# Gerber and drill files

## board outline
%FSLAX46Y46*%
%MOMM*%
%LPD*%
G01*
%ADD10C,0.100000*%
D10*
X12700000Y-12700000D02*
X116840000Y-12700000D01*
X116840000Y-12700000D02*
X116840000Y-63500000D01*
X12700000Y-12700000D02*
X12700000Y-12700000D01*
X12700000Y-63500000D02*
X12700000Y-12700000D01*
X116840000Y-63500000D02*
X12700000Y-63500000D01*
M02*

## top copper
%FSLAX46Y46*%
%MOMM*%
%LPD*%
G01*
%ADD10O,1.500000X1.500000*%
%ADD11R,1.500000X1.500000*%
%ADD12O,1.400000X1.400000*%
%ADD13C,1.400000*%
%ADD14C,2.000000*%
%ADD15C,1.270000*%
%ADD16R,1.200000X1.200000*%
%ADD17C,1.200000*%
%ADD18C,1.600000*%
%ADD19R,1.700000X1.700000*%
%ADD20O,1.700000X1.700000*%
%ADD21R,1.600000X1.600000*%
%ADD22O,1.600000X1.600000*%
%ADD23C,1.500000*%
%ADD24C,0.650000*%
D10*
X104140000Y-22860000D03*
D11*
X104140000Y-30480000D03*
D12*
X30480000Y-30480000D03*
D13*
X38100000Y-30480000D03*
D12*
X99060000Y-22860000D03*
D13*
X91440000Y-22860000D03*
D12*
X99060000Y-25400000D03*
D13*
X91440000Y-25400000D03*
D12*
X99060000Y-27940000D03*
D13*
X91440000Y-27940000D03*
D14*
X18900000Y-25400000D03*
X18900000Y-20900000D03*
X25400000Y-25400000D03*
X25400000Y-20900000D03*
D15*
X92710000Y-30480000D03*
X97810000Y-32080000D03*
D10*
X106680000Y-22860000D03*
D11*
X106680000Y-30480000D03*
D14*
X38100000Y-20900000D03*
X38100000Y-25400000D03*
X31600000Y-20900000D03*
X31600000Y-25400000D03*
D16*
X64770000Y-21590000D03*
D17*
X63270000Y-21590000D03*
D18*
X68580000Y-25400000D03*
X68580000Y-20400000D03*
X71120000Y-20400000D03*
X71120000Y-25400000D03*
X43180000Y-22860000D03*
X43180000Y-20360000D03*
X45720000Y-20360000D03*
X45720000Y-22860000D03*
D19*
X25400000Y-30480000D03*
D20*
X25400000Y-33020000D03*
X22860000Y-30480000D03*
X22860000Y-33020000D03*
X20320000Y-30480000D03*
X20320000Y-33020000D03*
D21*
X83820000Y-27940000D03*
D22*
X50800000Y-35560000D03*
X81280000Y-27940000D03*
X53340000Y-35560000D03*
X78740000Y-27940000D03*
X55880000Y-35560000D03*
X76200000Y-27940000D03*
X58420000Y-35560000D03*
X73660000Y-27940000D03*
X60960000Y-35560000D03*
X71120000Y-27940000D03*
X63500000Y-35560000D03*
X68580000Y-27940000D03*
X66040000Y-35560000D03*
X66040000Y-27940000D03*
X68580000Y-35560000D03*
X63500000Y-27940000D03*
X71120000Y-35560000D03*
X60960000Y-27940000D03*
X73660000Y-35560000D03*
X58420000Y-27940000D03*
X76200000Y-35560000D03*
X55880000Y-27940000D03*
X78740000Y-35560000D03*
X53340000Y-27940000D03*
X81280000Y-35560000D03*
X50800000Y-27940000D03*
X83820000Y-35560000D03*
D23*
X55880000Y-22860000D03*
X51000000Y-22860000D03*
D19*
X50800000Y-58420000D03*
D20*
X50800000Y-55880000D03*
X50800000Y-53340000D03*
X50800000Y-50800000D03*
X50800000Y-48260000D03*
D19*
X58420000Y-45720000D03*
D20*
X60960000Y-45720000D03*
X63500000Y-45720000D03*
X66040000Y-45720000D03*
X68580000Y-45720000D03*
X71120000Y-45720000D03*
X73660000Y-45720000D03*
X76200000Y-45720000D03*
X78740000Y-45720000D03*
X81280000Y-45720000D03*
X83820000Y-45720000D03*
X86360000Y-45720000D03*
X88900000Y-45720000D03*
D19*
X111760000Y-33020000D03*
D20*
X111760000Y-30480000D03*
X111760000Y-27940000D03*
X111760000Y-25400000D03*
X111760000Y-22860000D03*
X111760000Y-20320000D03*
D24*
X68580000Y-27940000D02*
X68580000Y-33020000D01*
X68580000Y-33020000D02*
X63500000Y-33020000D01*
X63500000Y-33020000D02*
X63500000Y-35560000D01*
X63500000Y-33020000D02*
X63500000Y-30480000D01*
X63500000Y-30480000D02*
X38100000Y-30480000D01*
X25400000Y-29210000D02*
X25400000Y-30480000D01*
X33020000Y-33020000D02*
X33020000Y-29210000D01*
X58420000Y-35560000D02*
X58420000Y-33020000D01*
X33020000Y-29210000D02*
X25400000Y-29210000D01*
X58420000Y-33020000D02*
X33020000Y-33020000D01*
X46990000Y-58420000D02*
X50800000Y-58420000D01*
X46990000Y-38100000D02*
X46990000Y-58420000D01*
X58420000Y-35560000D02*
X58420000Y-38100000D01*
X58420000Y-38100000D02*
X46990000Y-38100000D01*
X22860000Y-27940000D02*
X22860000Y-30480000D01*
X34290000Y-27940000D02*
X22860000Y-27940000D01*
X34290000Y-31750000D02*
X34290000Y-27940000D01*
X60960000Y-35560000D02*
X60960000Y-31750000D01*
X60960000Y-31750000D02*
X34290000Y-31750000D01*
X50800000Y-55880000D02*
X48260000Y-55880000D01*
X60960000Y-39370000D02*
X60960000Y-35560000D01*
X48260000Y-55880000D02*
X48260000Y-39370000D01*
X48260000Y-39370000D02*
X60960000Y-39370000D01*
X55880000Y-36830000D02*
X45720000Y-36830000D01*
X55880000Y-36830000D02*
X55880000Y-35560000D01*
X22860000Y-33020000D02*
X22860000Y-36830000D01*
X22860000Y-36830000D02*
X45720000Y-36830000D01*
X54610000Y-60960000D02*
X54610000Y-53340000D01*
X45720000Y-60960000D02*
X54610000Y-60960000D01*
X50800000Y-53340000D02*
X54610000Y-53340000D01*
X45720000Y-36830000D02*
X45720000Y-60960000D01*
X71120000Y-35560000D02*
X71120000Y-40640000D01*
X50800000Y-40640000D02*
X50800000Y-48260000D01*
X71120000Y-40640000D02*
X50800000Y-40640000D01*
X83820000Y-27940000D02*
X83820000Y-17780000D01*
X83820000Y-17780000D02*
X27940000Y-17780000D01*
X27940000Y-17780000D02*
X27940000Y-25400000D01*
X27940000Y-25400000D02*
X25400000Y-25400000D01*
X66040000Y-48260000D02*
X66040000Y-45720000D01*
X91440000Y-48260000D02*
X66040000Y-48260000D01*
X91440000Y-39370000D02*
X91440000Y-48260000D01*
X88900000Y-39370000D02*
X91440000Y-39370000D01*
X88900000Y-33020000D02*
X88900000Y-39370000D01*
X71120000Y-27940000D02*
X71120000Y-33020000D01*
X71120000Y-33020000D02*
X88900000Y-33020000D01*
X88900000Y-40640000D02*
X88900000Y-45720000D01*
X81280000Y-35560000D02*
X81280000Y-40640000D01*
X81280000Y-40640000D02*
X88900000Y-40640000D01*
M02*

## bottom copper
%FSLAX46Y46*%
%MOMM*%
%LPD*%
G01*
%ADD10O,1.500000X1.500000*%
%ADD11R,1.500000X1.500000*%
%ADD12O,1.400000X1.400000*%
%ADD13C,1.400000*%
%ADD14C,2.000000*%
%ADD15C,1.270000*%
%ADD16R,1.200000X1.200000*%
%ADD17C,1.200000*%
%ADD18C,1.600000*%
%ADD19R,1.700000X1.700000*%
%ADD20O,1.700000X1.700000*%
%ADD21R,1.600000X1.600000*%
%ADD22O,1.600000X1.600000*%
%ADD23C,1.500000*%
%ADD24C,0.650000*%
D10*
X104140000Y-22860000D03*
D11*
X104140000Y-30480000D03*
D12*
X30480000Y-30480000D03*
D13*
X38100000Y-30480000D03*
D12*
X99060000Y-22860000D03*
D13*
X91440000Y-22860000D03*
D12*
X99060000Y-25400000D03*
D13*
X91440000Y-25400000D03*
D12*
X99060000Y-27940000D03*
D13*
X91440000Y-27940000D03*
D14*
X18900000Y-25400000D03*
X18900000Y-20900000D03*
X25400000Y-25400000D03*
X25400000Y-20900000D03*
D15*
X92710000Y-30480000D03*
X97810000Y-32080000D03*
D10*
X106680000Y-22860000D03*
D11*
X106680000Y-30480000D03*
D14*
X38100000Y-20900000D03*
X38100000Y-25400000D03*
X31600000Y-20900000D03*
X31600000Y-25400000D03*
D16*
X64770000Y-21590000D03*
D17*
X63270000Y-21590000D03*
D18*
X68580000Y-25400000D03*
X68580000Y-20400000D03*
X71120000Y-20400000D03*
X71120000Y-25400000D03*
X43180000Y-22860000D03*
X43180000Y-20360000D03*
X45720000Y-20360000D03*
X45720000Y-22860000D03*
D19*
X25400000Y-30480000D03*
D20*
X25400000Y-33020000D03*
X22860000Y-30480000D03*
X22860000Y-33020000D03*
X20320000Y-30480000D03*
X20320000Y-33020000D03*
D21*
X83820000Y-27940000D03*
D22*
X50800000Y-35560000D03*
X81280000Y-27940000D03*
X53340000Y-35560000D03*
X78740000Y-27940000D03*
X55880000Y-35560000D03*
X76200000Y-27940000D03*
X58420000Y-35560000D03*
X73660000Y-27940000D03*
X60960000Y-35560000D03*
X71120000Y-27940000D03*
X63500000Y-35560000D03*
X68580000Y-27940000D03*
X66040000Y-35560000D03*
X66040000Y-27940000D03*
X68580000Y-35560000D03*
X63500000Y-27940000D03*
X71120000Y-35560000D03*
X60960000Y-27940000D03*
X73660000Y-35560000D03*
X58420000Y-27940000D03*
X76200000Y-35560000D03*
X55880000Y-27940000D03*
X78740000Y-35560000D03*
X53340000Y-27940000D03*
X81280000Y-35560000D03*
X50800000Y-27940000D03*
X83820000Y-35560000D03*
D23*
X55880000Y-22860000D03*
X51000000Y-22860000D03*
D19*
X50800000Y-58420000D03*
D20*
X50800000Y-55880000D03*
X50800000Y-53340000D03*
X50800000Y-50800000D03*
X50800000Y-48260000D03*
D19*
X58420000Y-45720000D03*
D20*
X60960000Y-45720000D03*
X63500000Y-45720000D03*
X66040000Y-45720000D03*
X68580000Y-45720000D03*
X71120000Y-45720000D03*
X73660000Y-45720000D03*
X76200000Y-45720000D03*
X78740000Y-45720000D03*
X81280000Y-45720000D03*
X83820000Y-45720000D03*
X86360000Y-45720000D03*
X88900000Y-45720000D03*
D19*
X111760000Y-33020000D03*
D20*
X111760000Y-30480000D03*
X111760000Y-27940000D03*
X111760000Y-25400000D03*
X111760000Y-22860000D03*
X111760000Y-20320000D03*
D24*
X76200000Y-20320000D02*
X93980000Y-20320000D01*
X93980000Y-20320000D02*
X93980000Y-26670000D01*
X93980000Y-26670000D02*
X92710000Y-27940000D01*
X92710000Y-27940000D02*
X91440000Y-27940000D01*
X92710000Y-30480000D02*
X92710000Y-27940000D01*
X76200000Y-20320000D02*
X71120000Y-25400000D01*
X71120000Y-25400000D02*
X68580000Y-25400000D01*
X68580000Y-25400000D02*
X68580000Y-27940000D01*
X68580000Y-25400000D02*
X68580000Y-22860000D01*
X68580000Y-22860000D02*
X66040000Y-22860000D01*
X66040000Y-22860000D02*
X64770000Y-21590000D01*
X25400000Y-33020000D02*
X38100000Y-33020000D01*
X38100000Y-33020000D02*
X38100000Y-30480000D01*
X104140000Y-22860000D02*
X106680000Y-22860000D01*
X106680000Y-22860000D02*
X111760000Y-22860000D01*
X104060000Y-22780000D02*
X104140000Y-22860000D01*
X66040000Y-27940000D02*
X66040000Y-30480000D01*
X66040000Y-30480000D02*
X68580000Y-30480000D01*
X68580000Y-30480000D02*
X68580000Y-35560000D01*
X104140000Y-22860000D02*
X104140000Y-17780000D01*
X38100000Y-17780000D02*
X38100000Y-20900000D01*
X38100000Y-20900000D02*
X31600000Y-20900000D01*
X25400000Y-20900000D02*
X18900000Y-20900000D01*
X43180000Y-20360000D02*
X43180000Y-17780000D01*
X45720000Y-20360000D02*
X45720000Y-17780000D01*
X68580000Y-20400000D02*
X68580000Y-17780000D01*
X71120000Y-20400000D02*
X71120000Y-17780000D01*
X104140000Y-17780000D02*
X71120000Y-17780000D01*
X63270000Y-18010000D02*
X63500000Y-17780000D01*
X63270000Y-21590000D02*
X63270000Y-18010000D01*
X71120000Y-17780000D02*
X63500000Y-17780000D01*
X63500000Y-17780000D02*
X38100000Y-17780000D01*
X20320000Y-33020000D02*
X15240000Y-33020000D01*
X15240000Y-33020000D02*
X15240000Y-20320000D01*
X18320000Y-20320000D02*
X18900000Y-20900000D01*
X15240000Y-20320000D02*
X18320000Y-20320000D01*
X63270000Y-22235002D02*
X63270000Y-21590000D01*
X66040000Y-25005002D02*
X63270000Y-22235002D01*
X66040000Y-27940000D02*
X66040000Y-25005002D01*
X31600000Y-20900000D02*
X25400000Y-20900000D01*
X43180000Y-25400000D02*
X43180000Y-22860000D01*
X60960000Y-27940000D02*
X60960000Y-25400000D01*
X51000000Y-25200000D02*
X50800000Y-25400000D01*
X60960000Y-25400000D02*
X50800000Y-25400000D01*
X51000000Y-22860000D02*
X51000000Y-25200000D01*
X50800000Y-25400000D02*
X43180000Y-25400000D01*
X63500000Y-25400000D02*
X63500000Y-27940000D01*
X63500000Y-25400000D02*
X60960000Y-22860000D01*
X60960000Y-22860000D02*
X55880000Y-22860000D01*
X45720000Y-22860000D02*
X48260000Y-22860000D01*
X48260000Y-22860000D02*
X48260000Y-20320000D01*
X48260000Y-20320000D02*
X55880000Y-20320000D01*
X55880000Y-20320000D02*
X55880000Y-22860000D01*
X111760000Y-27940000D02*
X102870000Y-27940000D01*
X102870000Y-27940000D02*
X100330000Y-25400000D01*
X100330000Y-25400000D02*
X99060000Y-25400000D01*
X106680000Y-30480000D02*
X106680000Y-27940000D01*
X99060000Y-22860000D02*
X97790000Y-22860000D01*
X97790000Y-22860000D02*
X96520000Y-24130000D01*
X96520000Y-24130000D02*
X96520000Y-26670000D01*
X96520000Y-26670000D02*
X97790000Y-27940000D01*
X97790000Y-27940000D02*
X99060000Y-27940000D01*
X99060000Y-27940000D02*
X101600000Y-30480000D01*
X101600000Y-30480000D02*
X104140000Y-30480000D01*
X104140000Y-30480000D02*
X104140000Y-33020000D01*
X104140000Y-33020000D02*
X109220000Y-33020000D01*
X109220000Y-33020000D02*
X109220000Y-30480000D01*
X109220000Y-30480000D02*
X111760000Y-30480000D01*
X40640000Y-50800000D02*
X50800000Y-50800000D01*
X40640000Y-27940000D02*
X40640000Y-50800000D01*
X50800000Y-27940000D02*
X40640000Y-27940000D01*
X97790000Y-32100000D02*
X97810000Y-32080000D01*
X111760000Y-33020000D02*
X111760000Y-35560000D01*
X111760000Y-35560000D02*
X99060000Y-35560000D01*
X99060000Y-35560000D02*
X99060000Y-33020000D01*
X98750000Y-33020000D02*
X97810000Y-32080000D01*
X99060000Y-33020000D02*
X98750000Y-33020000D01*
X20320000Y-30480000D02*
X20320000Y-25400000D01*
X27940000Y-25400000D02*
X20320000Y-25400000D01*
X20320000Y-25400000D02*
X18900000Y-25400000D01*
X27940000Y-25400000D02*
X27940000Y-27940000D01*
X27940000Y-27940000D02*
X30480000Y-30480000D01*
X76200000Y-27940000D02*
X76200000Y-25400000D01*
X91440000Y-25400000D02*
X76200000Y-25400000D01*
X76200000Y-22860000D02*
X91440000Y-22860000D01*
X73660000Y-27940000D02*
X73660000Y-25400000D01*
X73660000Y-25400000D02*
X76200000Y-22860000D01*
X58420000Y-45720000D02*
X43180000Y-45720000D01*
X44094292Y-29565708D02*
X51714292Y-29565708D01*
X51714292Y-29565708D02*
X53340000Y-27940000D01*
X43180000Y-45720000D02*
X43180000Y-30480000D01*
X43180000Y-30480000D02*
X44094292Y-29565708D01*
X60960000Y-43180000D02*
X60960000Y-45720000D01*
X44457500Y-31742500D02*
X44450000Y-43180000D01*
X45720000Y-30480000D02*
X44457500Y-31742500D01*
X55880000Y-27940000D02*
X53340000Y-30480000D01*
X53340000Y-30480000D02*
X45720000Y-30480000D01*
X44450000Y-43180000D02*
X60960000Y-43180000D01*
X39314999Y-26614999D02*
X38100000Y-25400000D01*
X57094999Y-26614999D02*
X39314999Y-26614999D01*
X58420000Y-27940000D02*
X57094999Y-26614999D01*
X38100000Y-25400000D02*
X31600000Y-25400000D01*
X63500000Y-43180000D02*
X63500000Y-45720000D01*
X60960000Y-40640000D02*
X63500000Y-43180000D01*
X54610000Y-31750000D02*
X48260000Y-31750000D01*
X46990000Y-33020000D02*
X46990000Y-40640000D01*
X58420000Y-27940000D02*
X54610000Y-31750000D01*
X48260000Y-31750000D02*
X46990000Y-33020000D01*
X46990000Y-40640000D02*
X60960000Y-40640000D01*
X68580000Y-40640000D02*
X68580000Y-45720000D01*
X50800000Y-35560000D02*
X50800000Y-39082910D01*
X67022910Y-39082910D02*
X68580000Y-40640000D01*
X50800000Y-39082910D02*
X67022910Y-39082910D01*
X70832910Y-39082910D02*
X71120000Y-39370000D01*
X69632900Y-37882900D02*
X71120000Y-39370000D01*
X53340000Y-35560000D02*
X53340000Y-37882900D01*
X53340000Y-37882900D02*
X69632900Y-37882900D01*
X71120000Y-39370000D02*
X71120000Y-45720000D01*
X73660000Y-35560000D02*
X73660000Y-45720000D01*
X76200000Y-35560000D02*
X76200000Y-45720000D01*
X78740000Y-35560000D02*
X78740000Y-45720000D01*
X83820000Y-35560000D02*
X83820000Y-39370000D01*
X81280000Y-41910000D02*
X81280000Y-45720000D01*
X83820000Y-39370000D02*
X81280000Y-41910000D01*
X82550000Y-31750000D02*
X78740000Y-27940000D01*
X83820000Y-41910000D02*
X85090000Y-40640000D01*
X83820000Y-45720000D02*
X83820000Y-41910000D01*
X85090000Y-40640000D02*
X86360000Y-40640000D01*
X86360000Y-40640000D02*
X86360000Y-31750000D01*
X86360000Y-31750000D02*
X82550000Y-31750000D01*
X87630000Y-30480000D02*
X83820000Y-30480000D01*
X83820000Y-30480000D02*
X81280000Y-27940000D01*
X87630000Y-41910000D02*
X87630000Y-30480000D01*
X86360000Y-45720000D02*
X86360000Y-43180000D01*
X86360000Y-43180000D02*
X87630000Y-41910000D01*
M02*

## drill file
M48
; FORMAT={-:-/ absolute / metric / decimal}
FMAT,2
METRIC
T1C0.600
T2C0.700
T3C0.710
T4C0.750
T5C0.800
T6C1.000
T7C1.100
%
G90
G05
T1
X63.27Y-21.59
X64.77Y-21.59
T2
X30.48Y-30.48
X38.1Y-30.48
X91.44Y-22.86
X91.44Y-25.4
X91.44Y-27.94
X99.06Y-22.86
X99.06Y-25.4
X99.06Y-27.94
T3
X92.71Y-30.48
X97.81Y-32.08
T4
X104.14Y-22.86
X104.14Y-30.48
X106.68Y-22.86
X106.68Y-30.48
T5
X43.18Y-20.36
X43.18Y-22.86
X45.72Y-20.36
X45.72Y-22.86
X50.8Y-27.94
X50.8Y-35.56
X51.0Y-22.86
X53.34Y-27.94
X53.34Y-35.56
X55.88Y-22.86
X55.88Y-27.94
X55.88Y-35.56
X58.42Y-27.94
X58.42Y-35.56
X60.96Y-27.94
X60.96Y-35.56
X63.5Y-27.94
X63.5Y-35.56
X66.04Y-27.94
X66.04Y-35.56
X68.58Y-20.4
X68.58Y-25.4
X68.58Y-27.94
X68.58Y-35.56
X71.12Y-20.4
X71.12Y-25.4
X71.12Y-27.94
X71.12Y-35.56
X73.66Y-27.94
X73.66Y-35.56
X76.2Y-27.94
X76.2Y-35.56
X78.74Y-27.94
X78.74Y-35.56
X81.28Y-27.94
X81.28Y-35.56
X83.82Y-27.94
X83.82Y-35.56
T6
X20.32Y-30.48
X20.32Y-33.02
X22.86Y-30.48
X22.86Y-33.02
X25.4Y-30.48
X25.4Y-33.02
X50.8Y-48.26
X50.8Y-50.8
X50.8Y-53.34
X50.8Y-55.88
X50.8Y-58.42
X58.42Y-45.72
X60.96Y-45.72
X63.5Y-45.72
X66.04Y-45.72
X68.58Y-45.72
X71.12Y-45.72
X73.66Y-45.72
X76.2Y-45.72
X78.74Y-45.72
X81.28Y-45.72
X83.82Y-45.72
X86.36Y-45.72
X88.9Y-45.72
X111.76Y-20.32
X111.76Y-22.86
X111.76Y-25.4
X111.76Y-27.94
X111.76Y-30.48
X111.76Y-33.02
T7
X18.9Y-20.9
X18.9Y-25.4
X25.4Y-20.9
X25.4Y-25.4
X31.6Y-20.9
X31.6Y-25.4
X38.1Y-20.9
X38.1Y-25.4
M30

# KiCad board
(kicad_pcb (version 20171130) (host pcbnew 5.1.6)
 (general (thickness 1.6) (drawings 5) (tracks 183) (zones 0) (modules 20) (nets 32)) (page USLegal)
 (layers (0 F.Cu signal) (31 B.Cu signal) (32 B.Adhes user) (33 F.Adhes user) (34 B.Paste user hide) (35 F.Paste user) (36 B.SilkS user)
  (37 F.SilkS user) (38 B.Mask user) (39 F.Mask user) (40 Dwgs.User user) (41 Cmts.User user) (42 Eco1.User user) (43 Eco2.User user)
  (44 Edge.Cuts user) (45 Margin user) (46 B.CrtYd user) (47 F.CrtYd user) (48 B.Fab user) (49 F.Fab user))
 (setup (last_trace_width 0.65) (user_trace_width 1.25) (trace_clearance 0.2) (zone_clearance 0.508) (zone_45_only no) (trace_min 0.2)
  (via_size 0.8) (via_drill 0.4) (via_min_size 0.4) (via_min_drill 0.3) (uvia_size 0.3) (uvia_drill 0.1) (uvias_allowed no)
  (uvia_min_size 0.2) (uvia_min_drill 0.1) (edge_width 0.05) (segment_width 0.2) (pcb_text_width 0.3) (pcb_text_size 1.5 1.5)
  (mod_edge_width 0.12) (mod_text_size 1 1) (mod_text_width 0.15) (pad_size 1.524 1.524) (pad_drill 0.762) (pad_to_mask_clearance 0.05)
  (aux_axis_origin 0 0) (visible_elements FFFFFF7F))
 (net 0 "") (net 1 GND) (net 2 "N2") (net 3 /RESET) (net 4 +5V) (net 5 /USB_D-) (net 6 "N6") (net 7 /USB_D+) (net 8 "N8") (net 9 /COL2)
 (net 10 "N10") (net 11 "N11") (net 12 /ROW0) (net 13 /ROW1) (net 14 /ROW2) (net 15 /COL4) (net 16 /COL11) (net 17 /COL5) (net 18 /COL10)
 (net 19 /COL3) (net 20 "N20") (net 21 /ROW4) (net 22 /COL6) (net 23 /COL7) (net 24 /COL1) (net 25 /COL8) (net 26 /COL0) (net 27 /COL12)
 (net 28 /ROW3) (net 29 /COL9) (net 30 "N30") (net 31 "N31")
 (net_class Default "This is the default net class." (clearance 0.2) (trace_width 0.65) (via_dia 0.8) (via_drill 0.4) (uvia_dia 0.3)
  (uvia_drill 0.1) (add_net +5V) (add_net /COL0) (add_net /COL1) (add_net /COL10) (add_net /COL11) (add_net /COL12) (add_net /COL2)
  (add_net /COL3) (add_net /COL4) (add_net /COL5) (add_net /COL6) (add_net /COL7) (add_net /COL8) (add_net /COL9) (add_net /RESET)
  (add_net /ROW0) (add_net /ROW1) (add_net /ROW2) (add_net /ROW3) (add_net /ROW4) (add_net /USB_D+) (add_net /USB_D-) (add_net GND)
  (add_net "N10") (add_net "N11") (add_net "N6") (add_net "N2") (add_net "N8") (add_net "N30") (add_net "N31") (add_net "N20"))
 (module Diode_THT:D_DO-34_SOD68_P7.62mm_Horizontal (layer F.Cu) (at 104.14 30.48 90)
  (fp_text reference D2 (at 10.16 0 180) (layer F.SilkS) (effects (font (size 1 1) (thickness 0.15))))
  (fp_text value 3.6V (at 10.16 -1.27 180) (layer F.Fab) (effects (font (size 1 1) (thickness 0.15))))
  (pad 2 thru_hole oval (at 7.62 0 90) (size 1.5 1.5) (drill 0.75) (layers *.Cu *.Mask) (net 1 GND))
  (pad 1 thru_hole rect (at 0 0 90) (size 1.5 1.5) (drill 0.75) (layers *.Cu *.Mask) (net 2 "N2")))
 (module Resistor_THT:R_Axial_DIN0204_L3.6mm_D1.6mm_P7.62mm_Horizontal (layer F.Cu) (at 38.1 30.48 180)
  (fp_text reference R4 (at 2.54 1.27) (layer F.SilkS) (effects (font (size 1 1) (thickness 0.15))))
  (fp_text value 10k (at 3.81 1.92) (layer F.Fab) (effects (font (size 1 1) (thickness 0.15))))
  (pad 2 thru_hole oval (at 7.62 0 180) (size 1.4 1.4) (drill 0.7) (layers *.Cu *.Mask) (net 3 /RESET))
  (pad 1 thru_hole circle (at 0 0 180) (size 1.4 1.4) (drill 0.7) (layers *.Cu *.Mask) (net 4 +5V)))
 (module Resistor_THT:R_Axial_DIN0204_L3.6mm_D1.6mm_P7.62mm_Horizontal (layer F.Cu) (at 91.44 22.86)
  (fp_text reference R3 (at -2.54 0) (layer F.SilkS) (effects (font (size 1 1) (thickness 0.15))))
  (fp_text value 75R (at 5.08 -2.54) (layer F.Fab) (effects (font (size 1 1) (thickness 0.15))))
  (pad 2 thru_hole oval (at 7.62 0) (size 1.4 1.4) (drill 0.7) (layers *.Cu *.Mask) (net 2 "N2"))
  (pad 1 thru_hole circle (at 0 0) (size 1.4 1.4) (drill 0.7) (layers *.Cu *.Mask) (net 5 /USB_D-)))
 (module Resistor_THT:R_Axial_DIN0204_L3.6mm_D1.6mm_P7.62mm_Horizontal (layer F.Cu) (at 91.44 25.4)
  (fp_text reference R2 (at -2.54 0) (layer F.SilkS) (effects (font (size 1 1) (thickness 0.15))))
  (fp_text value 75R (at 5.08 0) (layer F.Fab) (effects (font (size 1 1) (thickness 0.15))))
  (pad 2 thru_hole oval (at 7.62 0) (size 1.4 1.4) (drill 0.7) (layers *.Cu *.Mask) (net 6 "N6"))
  (pad 1 thru_hole circle (at 0 0) (size 1.4 1.4) (drill 0.7) (layers *.Cu *.Mask) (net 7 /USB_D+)))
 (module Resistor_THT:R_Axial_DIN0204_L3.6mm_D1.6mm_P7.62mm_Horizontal (layer F.Cu) (at 91.44 27.94)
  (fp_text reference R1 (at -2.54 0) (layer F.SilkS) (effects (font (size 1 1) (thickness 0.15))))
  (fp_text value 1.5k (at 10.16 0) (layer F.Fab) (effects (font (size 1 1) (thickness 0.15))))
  (pad 2 thru_hole oval (at 7.62 0) (size 1.4 1.4) (drill 0.7) (layers *.Cu *.Mask) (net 2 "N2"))
  (pad 1 thru_hole circle (at 0 0) (size 1.4 1.4) (drill 0.7) (layers *.Cu *.Mask) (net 4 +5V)))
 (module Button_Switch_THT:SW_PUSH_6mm (layer F.Cu) (at 25.4 25.4 180)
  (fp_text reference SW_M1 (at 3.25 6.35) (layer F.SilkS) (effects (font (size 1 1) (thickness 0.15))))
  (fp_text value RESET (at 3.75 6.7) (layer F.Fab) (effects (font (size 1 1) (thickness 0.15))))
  (pad 1 thru_hole circle (at 6.5 0 270) (size 2 2) (drill 1.1) (layers *.Cu *.Mask) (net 3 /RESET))
  (pad 2 thru_hole circle (at 6.5 4.5 270) (size 2 2) (drill 1.1) (layers *.Cu *.Mask) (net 1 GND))
  (pad 1 thru_hole circle (at 0 0 270) (size 2 2) (drill 1.1) (layers *.Cu *.Mask) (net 3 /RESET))
  (pad 2 thru_hole circle (at 0 4.5 270) (size 2 2) (drill 1.1) (layers *.Cu *.Mask) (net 1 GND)))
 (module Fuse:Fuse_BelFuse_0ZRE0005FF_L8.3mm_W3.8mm (layer F.Cu) (at 92.71 30.48)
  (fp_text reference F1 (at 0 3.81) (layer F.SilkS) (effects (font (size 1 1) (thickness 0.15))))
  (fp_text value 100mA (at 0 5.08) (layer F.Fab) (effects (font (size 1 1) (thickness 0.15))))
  (pad 1 thru_hole circle (at 0 0) (size 1.27 1.27) (drill 0.71) (layers *.Cu *.Mask) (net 4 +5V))
  (pad 2 thru_hole circle (at 5.1 1.6) (size 1.27 1.27) (drill 0.71) (layers *.Cu *.Mask) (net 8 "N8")))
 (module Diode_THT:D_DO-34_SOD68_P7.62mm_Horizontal (layer F.Cu) (at 106.68 30.48 90)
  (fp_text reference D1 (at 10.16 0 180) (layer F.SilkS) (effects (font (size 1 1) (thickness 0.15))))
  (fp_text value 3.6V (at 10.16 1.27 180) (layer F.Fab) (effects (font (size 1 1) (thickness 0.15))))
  (pad 2 thru_hole oval (at 7.62 0 90) (size 1.5 1.5) (drill 0.75) (layers *.Cu *.Mask) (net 1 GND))
  (pad 1 thru_hole rect (at 0 0 90) (size 1.5 1.5) (drill 0.75) (layers *.Cu *.Mask) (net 6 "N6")))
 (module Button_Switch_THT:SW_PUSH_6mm (layer F.Cu) (at 38.1 25.4 180)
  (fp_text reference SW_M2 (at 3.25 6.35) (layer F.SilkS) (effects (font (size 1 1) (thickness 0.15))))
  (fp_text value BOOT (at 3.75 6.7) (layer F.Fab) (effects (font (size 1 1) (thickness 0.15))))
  (pad 2 thru_hole circle (at 0 4.5 270) (size 2 2) (drill 1.1) (layers *.Cu *.Mask) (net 1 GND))
  (pad 1 thru_hole circle (at 0 0 270) (size 2 2) (drill 1.1) (layers *.Cu *.Mask) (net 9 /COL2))
  (pad 2 thru_hole circle (at 6.5 4.5 270) (size 2 2) (drill 1.1) (layers *.Cu *.Mask) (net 1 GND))
  (pad 1 thru_hole circle (at 6.5 0 270) (size 2 2) (drill 1.1) (layers *.Cu *.Mask) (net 9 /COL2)))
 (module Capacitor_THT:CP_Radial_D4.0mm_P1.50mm (layer F.Cu) (at 64.77 21.59 180)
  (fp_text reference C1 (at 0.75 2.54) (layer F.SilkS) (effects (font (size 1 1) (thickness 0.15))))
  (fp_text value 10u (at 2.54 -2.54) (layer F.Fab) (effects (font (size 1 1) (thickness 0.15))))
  (pad 1 thru_hole rect (at 0 0 180) (size 1.2 1.2) (drill 0.6) (layers *.Cu *.Mask) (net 4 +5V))
  (pad 2 thru_hole circle (at 1.5 0 180) (size 1.2 1.2) (drill 0.6) (layers *.Cu *.Mask) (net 1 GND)))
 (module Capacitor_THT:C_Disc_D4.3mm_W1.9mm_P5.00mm (layer F.Cu) (at 68.58 25.4 90)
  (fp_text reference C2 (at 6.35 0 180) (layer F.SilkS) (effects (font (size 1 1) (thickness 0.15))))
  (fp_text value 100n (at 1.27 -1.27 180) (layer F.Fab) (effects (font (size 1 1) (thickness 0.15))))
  (pad 1 thru_hole circle (at 0 0 90) (size 1.6 1.6) (drill 0.8) (layers *.Cu *.Mask) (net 4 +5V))
  (pad 2 thru_hole circle (at 5 0 90) (size 1.6 1.6) (drill 0.8) (layers *.Cu *.Mask) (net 1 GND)))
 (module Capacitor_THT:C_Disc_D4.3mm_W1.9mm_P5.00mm (layer F.Cu) (at 71.12 25.4 90)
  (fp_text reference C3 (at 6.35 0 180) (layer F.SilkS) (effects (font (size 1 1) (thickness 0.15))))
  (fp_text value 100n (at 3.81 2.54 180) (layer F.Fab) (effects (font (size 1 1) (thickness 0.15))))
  (pad 2 thru_hole circle (at 5 0 90) (size 1.6 1.6) (drill 0.8) (layers *.Cu *.Mask) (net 1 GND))
  (pad 1 thru_hole circle (at 0 0 90) (size 1.6 1.6) (drill 0.8) (layers *.Cu *.Mask) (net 4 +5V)))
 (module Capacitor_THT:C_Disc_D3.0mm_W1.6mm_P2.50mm (layer F.Cu) (at 43.18 22.86 90)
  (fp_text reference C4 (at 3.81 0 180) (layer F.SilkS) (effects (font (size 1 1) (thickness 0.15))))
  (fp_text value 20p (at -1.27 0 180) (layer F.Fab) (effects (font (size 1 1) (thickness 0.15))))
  (pad 1 thru_hole circle (at 0 0 90) (size 1.6 1.6) (drill 0.8) (layers *.Cu *.Mask) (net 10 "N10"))
  (pad 2 thru_hole circle (at 2.5 0 90) (size 1.6 1.6) (drill 0.8) (layers *.Cu *.Mask) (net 1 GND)))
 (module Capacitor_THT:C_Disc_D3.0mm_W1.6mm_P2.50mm (layer F.Cu) (at 45.72 22.86 90)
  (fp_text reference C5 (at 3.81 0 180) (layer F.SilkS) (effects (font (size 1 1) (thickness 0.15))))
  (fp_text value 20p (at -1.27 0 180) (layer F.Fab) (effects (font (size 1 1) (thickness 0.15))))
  (pad 2 thru_hole circle (at 2.5 0 90) (size 1.6 1.6) (drill 0.8) (layers *.Cu *.Mask) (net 1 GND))
  (pad 1 thru_hole circle (at 0 0 90) (size 1.6 1.6) (drill 0.8) (layers *.Cu *.Mask) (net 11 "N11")))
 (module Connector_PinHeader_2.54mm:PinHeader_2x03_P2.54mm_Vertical (layer F.Cu) (at 25.4 30.48 270)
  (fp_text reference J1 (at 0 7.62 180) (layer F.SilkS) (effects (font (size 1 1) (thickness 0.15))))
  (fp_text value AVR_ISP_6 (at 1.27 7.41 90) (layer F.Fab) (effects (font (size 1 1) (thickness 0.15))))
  (pad 1 thru_hole rect (at 0 0 270) (size 1.7 1.7) (drill 1) (layers *.Cu *.Mask) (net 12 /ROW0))
  (pad 2 thru_hole oval (at 2.54 0 270) (size 1.7 1.7) (drill 1) (layers *.Cu *.Mask) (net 4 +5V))
  (pad 3 thru_hole oval (at 0 2.54 270) (size 1.7 1.7) (drill 1) (layers *.Cu *.Mask) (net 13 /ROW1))
  (pad 4 thru_hole oval (at 2.54 2.54 270) (size 1.7 1.7) (drill 1) (layers *.Cu *.Mask) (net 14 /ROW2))
  (pad 5 thru_hole oval (at 0 5.08 270) (size 1.7 1.7) (drill 1) (layers *.Cu *.Mask) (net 3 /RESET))
  (pad 6 thru_hole oval (at 2.54 5.08 270) (size 1.7 1.7) (drill 1) (layers *.Cu *.Mask) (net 1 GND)))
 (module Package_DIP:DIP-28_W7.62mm (layer F.Cu) (at 83.82 27.94 270)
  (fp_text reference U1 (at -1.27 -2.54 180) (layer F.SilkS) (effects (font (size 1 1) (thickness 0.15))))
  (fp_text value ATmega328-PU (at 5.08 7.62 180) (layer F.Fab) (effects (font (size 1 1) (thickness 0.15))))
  (pad 1 thru_hole rect (at 0 0 270) (size 1.6 1.6) (drill 0.8) (layers *.Cu *.Mask) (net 3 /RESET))
  (pad 15 thru_hole oval (at 7.62 33.02 270) (size 1.6 1.6) (drill 0.8) (layers *.Cu *.Mask) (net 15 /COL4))
  (pad 2 thru_hole oval (at 0 2.54 270) (size 1.6 1.6) (drill 0.8) (layers *.Cu *.Mask) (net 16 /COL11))
  (pad 16 thru_hole oval (at 7.62 30.48 270) (size 1.6 1.6) (drill 0.8) (layers *.Cu *.Mask) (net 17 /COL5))
  (pad 3 thru_hole oval (at 0 5.08 270) (size 1.6 1.6) (drill 0.8) (layers *.Cu *.Mask) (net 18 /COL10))
  (pad 17 thru_hole oval (at 7.62 27.94 270) (size 1.6 1.6) (drill 0.8) (layers *.Cu *.Mask) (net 14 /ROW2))
  (pad 4 thru_hole oval (at 0 7.62 270) (size 1.6 1.6) (drill 0.8) (layers *.Cu *.Mask) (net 7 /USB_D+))
  (pad 18 thru_hole oval (at 7.62 25.4 270) (size 1.6 1.6) (drill 0.8) (layers *.Cu *.Mask) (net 12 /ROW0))
  (pad 5 thru_hole oval (at 0 10.16 270) (size 1.6 1.6) (drill 0.8) (layers *.Cu *.Mask) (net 5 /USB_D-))
  (pad 19 thru_hole oval (at 7.62 22.86 270) (size 1.6 1.6) (drill 0.8) (layers *.Cu *.Mask) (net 13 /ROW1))
  (pad 6 thru_hole oval (at 0 12.7 270) (size 1.6 1.6) (drill 0.8) (layers *.Cu *.Mask) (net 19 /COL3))
  (pad 20 thru_hole oval (at 7.62 20.32 270) (size 1.6 1.6) (drill 0.8) (layers *.Cu *.Mask) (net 4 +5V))
  (pad 7 thru_hole oval (at 0 15.24 270) (size 1.6 1.6) (drill 0.8) (layers *.Cu *.Mask) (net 4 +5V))
  (pad 21 thru_hole oval (at 7.62 17.78 270) (size 1.6 1.6) (drill 0.8) (layers *.Cu *.Mask) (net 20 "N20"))
  (pad 8 thru_hole oval (at 0 17.78 270) (size 1.6 1.6) (drill 0.8) (layers *.Cu *.Mask) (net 1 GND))
  (pad 22 thru_hole oval (at 7.62 15.24 270) (size 1.6 1.6) (drill 0.8) (layers *.Cu *.Mask) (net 1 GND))
  (pad 9 thru_hole oval (at 0 20.32 270) (size 1.6 1.6) (drill 0.8) (layers *.Cu *.Mask) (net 11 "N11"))
  (pad 23 thru_hole oval (at 7.62 12.7 270) (size 1.6 1.6) (drill 0.8) (layers *.Cu *.Mask) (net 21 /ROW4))
  (pad 10 thru_hole oval (at 0 22.86 270) (size 1.6 1.6) (drill 0.8) (layers *.Cu *.Mask) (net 10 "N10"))
  (pad 24 thru_hole oval (at 7.62 10.16 270) (size 1.6 1.6) (drill 0.8) (layers *.Cu *.Mask) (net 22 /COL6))
  (pad 11 thru_hole oval (at 0 25.4 270) (size 1.6 1.6) (drill 0.8) (layers *.Cu *.Mask) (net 9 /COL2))
  (pad 25 thru_hole oval (at 7.62 7.62 270) (size 1.6 1.6) (drill 0.8) (layers *.Cu *.Mask) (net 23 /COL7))
  (pad 12 thru_hole oval (at 0 27.94 270) (size 1.6 1.6) (drill 0.8) (layers *.Cu *.Mask) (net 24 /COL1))
  (pad 26 thru_hole oval (at 7.62 5.08 270) (size 1.6 1.6) (drill 0.8) (layers *.Cu *.Mask) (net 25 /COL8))
  (pad 13 thru_hole oval (at 0 30.48 270) (size 1.6 1.6) (drill 0.8) (layers *.Cu *.Mask) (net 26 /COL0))
  (pad 27 thru_hole oval (at 7.62 2.54 270) (size 1.6 1.6) (drill 0.8) (layers *.Cu *.Mask) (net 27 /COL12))
  (pad 14 thru_hole oval (at 0 33.02 270) (size 1.6 1.6) (drill 0.8) (layers *.Cu *.Mask) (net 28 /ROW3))
  (pad 28 thru_hole oval (at 7.62 0 270) (size 1.6 1.6) (drill 0.8) (layers *.Cu *.Mask) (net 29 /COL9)))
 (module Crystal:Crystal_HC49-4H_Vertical (layer F.Cu) (at 55.88 22.86 180)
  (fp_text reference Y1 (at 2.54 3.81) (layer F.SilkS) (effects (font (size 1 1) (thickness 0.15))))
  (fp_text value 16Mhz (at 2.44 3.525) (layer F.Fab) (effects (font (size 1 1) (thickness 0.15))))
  (pad 1 thru_hole circle (at 0 0 180) (size 1.5 1.5) (drill 0.8) (layers *.Cu *.Mask) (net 11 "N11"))
  (pad 2 thru_hole circle (at 4.88 0 180) (size 1.5 1.5) (drill 0.8) (layers *.Cu *.Mask) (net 10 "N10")))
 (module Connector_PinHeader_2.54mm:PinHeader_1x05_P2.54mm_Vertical (layer F.Cu) (at 50.8 58.42 180)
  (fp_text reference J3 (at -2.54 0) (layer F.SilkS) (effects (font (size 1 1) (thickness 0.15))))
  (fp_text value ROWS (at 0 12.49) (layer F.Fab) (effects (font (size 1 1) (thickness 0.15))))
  (pad 1 thru_hole rect (at 0 0 180) (size 1.7 1.7) (drill 1) (layers *.Cu *.Mask) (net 12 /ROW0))
  (pad 2 thru_hole oval (at 0 2.54 180) (size 1.7 1.7) (drill 1) (layers *.Cu *.Mask) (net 13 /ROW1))
  (pad 3 thru_hole oval (at 0 5.08 180) (size 1.7 1.7) (drill 1) (layers *.Cu *.Mask) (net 14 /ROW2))
  (pad 4 thru_hole oval (at 0 7.62 180) (size 1.7 1.7) (drill 1) (layers *.Cu *.Mask) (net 28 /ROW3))
  (pad 5 thru_hole oval (at 0 10.16 180) (size 1.7 1.7) (drill 1) (layers *.Cu *.Mask) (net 21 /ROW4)))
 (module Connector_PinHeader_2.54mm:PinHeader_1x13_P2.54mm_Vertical (layer F.Cu) (at 58.42 45.72 90)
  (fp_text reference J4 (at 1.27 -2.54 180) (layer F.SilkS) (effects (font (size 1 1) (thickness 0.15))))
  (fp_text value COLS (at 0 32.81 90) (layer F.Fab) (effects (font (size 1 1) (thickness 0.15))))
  (pad 1 thru_hole rect (at 0 0 90) (size 1.7 1.7) (drill 1) (layers *.Cu *.Mask) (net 26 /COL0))
  (pad 2 thru_hole oval (at 0 2.54 90) (size 1.7 1.7) (drill 1) (layers *.Cu *.Mask) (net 24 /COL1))
  (pad 3 thru_hole oval (at 0 5.08 90) (size 1.7 1.7) (drill 1) (layers *.Cu *.Mask) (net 9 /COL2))
  (pad 4 thru_hole oval (at 0 7.62 90) (size 1.7 1.7) (drill 1) (layers *.Cu *.Mask) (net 19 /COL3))
  (pad 5 thru_hole oval (at 0 10.16 90) (size 1.7 1.7) (drill 1) (layers *.Cu *.Mask) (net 15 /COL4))
  (pad 6 thru_hole oval (at 0 12.7 90) (size 1.7 1.7) (drill 1) (layers *.Cu *.Mask) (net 17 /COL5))
  (pad 7 thru_hole oval (at 0 15.24 90) (size 1.7 1.7) (drill 1) (layers *.Cu *.Mask) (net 22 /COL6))
  (pad 8 thru_hole oval (at 0 17.78 90) (size 1.7 1.7) (drill 1) (layers *.Cu *.Mask) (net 23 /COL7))
  (pad 9 thru_hole oval (at 0 20.32 90) (size 1.7 1.7) (drill 1) (layers *.Cu *.Mask) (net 25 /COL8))
  (pad 10 thru_hole oval (at 0 22.86 90) (size 1.7 1.7) (drill 1) (layers *.Cu *.Mask) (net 29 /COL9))
  (pad 11 thru_hole oval (at 0 25.4 90) (size 1.7 1.7) (drill 1) (layers *.Cu *.Mask) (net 18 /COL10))
  (pad 12 thru_hole oval (at 0 27.94 90) (size 1.7 1.7) (drill 1) (layers *.Cu *.Mask) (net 16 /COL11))
  (pad 13 thru_hole oval (at 0 30.48 90) (size 1.7 1.7) (drill 1) (layers *.Cu *.Mask) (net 27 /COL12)))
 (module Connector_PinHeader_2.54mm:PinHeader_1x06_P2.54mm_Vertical (layer F.Cu) (at 111.76 33.02 180)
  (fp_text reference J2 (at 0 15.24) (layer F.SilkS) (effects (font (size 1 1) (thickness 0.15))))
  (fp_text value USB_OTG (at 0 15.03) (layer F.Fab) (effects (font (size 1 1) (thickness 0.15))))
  (pad 1 thru_hole rect (at 0 0 180) (size 1.7 1.7) (drill 1) (layers *.Cu *.Mask) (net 8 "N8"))
  (pad 2 thru_hole oval (at 0 2.54 180) (size 1.7 1.7) (drill 1) (layers *.Cu *.Mask) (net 2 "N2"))
  (pad 3 thru_hole oval (at 0 5.08 180) (size 1.7 1.7) (drill 1) (layers *.Cu *.Mask) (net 6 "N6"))
  (pad 4 thru_hole oval (at 0 7.62 180) (size 1.7 1.7) (drill 1) (layers *.Cu *.Mask) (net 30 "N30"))
  (pad 5 thru_hole oval (at 0 10.16 180) (size 1.7 1.7) (drill 1) (layers *.Cu *.Mask) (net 1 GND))
  (pad 6 thru_hole oval (at 0 12.7 180) (size 1.7 1.7) (drill 1) (layers *.Cu *.Mask) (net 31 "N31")))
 (gr_line (start 12.7 12.7) (end 116.84 12.7) (layer Edge.Cuts) (width 0.1))
 (gr_line (start 116.84 12.7) (end 116.84 63.5) (layer Edge.Cuts) (width 0.1))
 (gr_line (start 12.7 12.7) (end 12.7 12.7) (layer Edge.Cuts) (width 0.1))
 (gr_line (start 12.7 63.5) (end 12.7 12.7) (layer Edge.Cuts) (width 0.1))
 (gr_line (start 116.84 63.5) (end 12.7 63.5) (layer Edge.Cuts) (width 0.1))
 (segment (start 76.2 20.32) (end 93.98 20.32) (width 0.65) (layer B.Cu) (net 4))
 (segment (start 93.98 20.32) (end 93.98 26.67) (width 0.65) (layer B.Cu) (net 4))
 (segment (start 93.98 26.67) (end 92.71 27.94) (width 0.65) (layer B.Cu) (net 4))
 (segment (start 92.71 27.94) (end 91.44 27.94) (width 0.65) (layer B.Cu) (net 4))
 (segment (start 92.71 30.48) (end 92.71 27.94) (width 0.65) (layer B.Cu) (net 4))
 (segment (start 76.2 20.32) (end 71.12 25.4) (width 0.65) (layer B.Cu) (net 4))
 (segment (start 71.12 25.4) (end 68.58 25.4) (width 0.65) (layer B.Cu) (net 4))
 (segment (start 68.58 27.94) (end 68.58 33.02) (width 0.65) (layer F.Cu) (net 4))
 (segment (start 68.58 33.02) (end 63.5 33.02) (width 0.65) (layer F.Cu) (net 4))
 (segment (start 63.5 33.02) (end 63.5 35.56) (width 0.65) (layer F.Cu) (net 4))
 (segment (start 68.58 25.4) (end 68.58 27.94) (width 0.65) (layer B.Cu) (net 4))
 (segment (start 68.58 25.4) (end 68.58 22.86) (width 0.65) (layer B.Cu) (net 4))
 (segment (start 68.58 22.86) (end 66.04 22.86) (width 0.65) (layer B.Cu) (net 4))
 (segment (start 66.04 22.86) (end 64.77 21.59) (width 0.65) (layer B.Cu) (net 4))
 (segment (start 63.5 33.02) (end 63.5 30.48) (width 0.65) (layer F.Cu) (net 4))
 (segment (start 63.5 30.48) (end 38.1 30.48) (width 0.65) (layer F.Cu) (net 4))
 (segment (start 25.4 33.02) (end 38.1 33.02) (width 0.65) (layer B.Cu) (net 4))
 (segment (start 38.1 33.02) (end 38.1 30.48) (width 0.65) (layer B.Cu) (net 4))
 (segment (start 104.14 22.86) (end 106.68 22.86) (width 0.65) (layer B.Cu) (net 1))
 (segment (start 106.68 22.86) (end 111.76 22.86) (width 0.65) (layer B.Cu) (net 1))
 (segment (start 104.06 22.78) (end 104.14 22.86) (width 0.65) (layer B.Cu) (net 1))
 (segment (start 66.04 27.94) (end 66.04 30.48) (width 0.65) (layer B.Cu) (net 1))
 (segment (start 66.04 30.48) (end 68.58 30.48) (width 0.65) (layer B.Cu) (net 1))
 (segment (start 68.58 30.48) (end 68.58 35.56) (width 0.65) (layer B.Cu) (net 1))
 (segment (start 104.14 22.86) (end 104.14 17.78) (width 0.65) (layer B.Cu) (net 1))
 (segment (start 38.1 17.78) (end 38.1 20.9) (width 0.65) (layer B.Cu) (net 1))
 (segment (start 38.1 20.9) (end 31.6 20.9) (width 0.65) (layer B.Cu) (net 1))
 (segment (start 25.4 20.9) (end 18.9 20.9) (width 0.65) (layer B.Cu) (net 1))
 (segment (start 43.18 20.36) (end 43.18 17.78) (width 0.65) (layer B.Cu) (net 1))
 (segment (start 45.72 20.36) (end 45.72 17.78) (width 0.65) (layer B.Cu) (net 1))
 (segment (start 68.58 20.4) (end 68.58 17.78) (width 0.65) (layer B.Cu) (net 1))
 (segment (start 71.12 20.4) (end 71.12 17.78) (width 0.65) (layer B.Cu) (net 1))
 (segment (start 104.14 17.78) (end 71.12 17.78) (width 0.65) (layer B.Cu) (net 1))
 (segment (start 63.27 18.01) (end 63.5 17.78) (width 0.65) (layer B.Cu) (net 1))
 (segment (start 63.27 21.59) (end 63.27 18.01) (width 0.65) (layer B.Cu) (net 1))
 (segment (start 71.12 17.78) (end 63.5 17.78) (width 0.65) (layer B.Cu) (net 1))
 (segment (start 63.5 17.78) (end 38.1 17.78) (width 0.65) (layer B.Cu) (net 1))
 (segment (start 20.32 33.02) (end 15.24 33.02) (width 0.65) (layer B.Cu) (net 1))
 (segment (start 15.24 33.02) (end 15.24 20.32) (width 0.65) (layer B.Cu) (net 1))
 (segment (start 18.32 20.32) (end 18.9 20.9) (width 0.65) (layer B.Cu) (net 1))
 (segment (start 15.24 20.32) (end 18.32 20.32) (width 0.65) (layer B.Cu) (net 1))
 (segment (start 63.27 22.235002) (end 63.27 21.59) (width 0.65) (layer B.Cu) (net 1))
 (segment (start 66.04 25.005002) (end 63.27 22.235002) (width 0.65) (layer B.Cu) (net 1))
 (segment (start 66.04 27.94) (end 66.04 25.005002) (width 0.65) (layer B.Cu) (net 1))
 (segment (start 31.6 20.9) (end 25.4 20.9) (width 0.65) (layer B.Cu) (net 1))
 (segment (start 43.18 25.4) (end 43.18 22.86) (width 0.65) (layer B.Cu) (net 10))
 (segment (start 60.96 27.94) (end 60.96 25.4) (width 0.65) (layer B.Cu) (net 10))
 (segment (start 51 25.2) (end 50.8 25.4) (width 0.65) (layer B.Cu) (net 10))
 (segment (start 60.96 25.4) (end 50.8 25.4) (width 0.65) (layer B.Cu) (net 10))
 (segment (start 51 22.86) (end 51 25.2) (width 0.65) (layer B.Cu) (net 10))
 (segment (start 50.8 25.4) (end 43.18 25.4) (width 0.65) (layer B.Cu) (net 10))
 (segment (start 63.5 25.4) (end 63.5 27.94) (width 0.65) (layer B.Cu) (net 11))
 (segment (start 63.5 25.4) (end 60.96 22.86) (width 0.65) (layer B.Cu) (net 11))
 (segment (start 60.96 22.86) (end 55.88 22.86) (width 0.65) (layer B.Cu) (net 11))
 (segment (start 45.72 22.86) (end 48.26 22.86) (width 0.65) (layer B.Cu) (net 11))
 (segment (start 48.26 22.86) (end 48.26 20.32) (width 0.65) (layer B.Cu) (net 11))
 (segment (start 48.26 20.32) (end 55.88 20.32) (width 0.65) (layer B.Cu) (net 11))
 (segment (start 55.88 20.32) (end 55.88 22.86) (width 0.65) (layer B.Cu) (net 11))
 (segment (start 111.76 27.94) (end 102.87 27.94) (width 0.65) (layer B.Cu) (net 6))
 (segment (start 102.87 27.94) (end 100.33 25.4) (width 0.65) (layer B.Cu) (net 6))
 (segment (start 100.33 25.4) (end 99.06 25.4) (width 0.65) (layer B.Cu) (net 6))
 (segment (start 106.68 30.48) (end 106.68 27.94) (width 0.65) (layer B.Cu) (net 6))
 (segment (start 99.06 22.86) (end 97.79 22.86) (width 0.65) (layer B.Cu) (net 2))
 (segment (start 97.79 22.86) (end 96.52 24.13) (width 0.65) (layer B.Cu) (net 2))
 (segment (start 96.52 24.13) (end 96.52 26.67) (width 0.65) (layer B.Cu) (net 2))
 (segment (start 96.52 26.67) (end 97.79 27.94) (width 0.65) (layer B.Cu) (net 2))
 (segment (start 97.79 27.94) (end 99.06 27.94) (width 0.65) (layer B.Cu) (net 2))
 (segment (start 99.06 27.94) (end 101.6 30.48) (width 0.65) (layer B.Cu) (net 2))
 (segment (start 101.6 30.48) (end 104.14 30.48) (width 0.65) (layer B.Cu) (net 2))
 (segment (start 104.14 30.48) (end 104.14 33.02) (width 0.65) (layer B.Cu) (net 2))
 (segment (start 104.14 33.02) (end 109.22 33.02) (width 0.65) (layer B.Cu) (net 2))
 (segment (start 109.22 33.02) (end 109.22 30.48) (width 0.65) (layer B.Cu) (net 2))
 (segment (start 109.22 30.48) (end 111.76 30.48) (width 0.65) (layer B.Cu) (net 2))
 (segment (start 25.4 29.21) (end 25.4 30.48) (width 0.65) (layer F.Cu) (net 12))
 (segment (start 33.02 33.02) (end 33.02 29.21) (width 0.65) (layer F.Cu) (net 12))
 (segment (start 58.42 35.56) (end 58.42 33.02) (width 0.65) (layer F.Cu) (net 12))
 (segment (start 33.02 29.21) (end 25.4 29.21) (width 0.65) (layer F.Cu) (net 12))
 (segment (start 58.42 33.02) (end 33.02 33.02) (width 0.65) (layer F.Cu) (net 12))
 (segment (start 46.99 58.42) (end 50.8 58.42) (width 0.65) (layer F.Cu) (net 12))
 (segment (start 46.99 38.1) (end 46.99 58.42) (width 0.65) (layer F.Cu) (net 12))
 (segment (start 58.42 35.56) (end 58.42 38.1) (width 0.65) (layer F.Cu) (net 12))
 (segment (start 58.42 38.1) (end 46.99 38.1) (width 0.65) (layer F.Cu) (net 12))
 (segment (start 22.86 27.94) (end 22.86 30.48) (width 0.65) (layer F.Cu) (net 13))
 (segment (start 34.29 27.94) (end 22.86 27.94) (width 0.65) (layer F.Cu) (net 13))
 (segment (start 34.29 31.75) (end 34.29 27.94) (width 0.65) (layer F.Cu) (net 13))
 (segment (start 60.96 35.56) (end 60.96 31.75) (width 0.65) (layer F.Cu) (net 13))
 (segment (start 60.96 31.75) (end 34.29 31.75) (width 0.65) (layer F.Cu) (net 13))
 (segment (start 50.8 55.88) (end 48.26 55.88) (width 0.65) (layer F.Cu) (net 13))
 (segment (start 60.96 39.37) (end 60.96 35.56) (width 0.65) (layer F.Cu) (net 13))
 (segment (start 48.26 55.88) (end 48.26 39.37) (width 0.65) (layer F.Cu) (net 13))
 (segment (start 48.26 39.37) (end 60.96 39.37) (width 0.65) (layer F.Cu) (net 13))
 (segment (start 55.88 36.83) (end 45.72 36.83) (width 0.65) (layer F.Cu) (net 14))
 (segment (start 55.88 36.83) (end 55.88 35.56) (width 0.65) (layer F.Cu) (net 14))
 (segment (start 22.86 33.02) (end 22.86 36.83) (width 0.65) (layer F.Cu) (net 14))
 (segment (start 22.86 36.83) (end 45.72 36.83) (width 0.65) (layer F.Cu) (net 14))
 (segment (start 54.61 60.96) (end 54.61 53.34) (width 0.65) (layer F.Cu) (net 14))
 (segment (start 45.72 60.96) (end 54.61 60.96) (width 0.65) (layer F.Cu) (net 14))
 (segment (start 50.8 53.34) (end 54.61 53.34) (width 0.65) (layer F.Cu) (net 14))
 (segment (start 45.72 36.83) (end 45.72 60.96) (width 0.65) (layer F.Cu) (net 14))
 (segment (start 40.64 50.8) (end 50.8 50.8) (width 0.65) (layer B.Cu) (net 28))
 (segment (start 40.64 27.94) (end 40.64 50.8) (width 0.65) (layer B.Cu) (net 28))
 (segment (start 50.8 27.94) (end 40.64 27.94) (width 0.65) (layer B.Cu) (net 28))
 (segment (start 71.12 35.56) (end 71.12 40.64) (width 0.65) (layer F.Cu) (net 21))
 (segment (start 50.8 40.64) (end 50.8 48.26) (width 0.65) (layer F.Cu) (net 21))
 (segment (start 71.12 40.64) (end 50.8 40.64) (width 0.65) (layer F.Cu) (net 21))
 (segment (start 97.79 32.1) (end 97.81 32.08) (width 0.65) (layer B.Cu) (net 8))
 (segment (start 111.76 33.02) (end 111.76 35.56) (width 0.65) (layer B.Cu) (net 8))
 (segment (start 111.76 35.56) (end 99.06 35.56) (width 0.65) (layer B.Cu) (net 8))
 (segment (start 99.06 35.56) (end 99.06 33.02) (width 0.65) (layer B.Cu) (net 8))
 (segment (start 98.75 33.02) (end 97.81 32.08) (width 0.65) (layer B.Cu) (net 8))
 (segment (start 99.06 33.02) (end 98.75 33.02) (width 0.65) (layer B.Cu) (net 8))
 (segment (start 20.32 30.48) (end 20.32 25.4) (width 0.65) (layer B.Cu) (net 3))
 (segment (start 27.94 25.4) (end 20.32 25.4) (width 0.65) (layer B.Cu) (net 3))
 (segment (start 20.32 25.4) (end 18.9 25.4) (width 0.65) (layer B.Cu) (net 3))
 (segment (start 27.94 25.4) (end 27.94 27.94) (width 0.65) (layer B.Cu) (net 3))
 (segment (start 27.94 27.94) (end 30.48 30.48) (width 0.65) (layer B.Cu) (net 3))
 (segment (start 83.82 27.94) (end 83.82 17.78) (width 0.65) (layer F.Cu) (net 3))
 (segment (start 83.82 17.78) (end 27.94 17.78) (width 0.65) (layer F.Cu) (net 3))
 (segment (start 27.94 17.78) (end 27.94 25.4) (width 0.65) (layer F.Cu) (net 3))
 (segment (start 27.94 25.4) (end 25.4 25.4) (width 0.65) (layer F.Cu) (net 3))
 (segment (start 76.2 27.94) (end 76.2 25.4) (width 0.65) (layer B.Cu) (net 7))
 (segment (start 91.44 25.4) (end 76.2 25.4) (width 0.65) (layer B.Cu) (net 7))
 (segment (start 76.2 22.86) (end 91.44 22.86) (width 0.65) (layer B.Cu) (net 5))
 (segment (start 73.66 27.94) (end 73.66 25.4) (width 0.65) (layer B.Cu) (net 5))
 (segment (start 73.66 25.4) (end 76.2 22.86) (width 0.65) (layer B.Cu) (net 5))
 (segment (start 58.42 45.72) (end 43.18 45.72) (width 0.65) (layer B.Cu) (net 26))
 (segment (start 44.094292 29.565708) (end 51.714292 29.565708) (width 0.65) (layer B.Cu) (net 26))
 (segment (start 51.714292 29.565708) (end 53.34 27.94) (width 0.65) (layer B.Cu) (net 26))
 (segment (start 43.18 45.72) (end 43.18 30.48) (width 0.65) (layer B.Cu) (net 26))
 (segment (start 43.18 30.48) (end 44.094292 29.565708) (width 0.65) (layer B.Cu) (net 26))
 (segment (start 60.96 43.18) (end 60.96 45.72) (width 0.65) (layer B.Cu) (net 24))
 (segment (start 44.4575 31.7425) (end 44.45 43.18) (width 0.65) (layer B.Cu) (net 24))
 (segment (start 45.72 30.48) (end 44.4575 31.7425) (width 0.65) (layer B.Cu) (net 24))
 (segment (start 55.88 27.94) (end 53.34 30.48) (width 0.65) (layer B.Cu) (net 24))
 (segment (start 53.34 30.48) (end 45.72 30.48) (width 0.65) (layer B.Cu) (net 24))
 (segment (start 44.45 43.18) (end 60.96 43.18) (width 0.65) (layer B.Cu) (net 24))
 (segment (start 39.314999 26.614999) (end 38.1 25.4) (width 0.65) (layer B.Cu) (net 9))
 (segment (start 57.094999 26.614999) (end 39.314999 26.614999) (width 0.65) (layer B.Cu) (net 9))
 (segment (start 58.42 27.94) (end 57.094999 26.614999) (width 0.65) (layer B.Cu) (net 9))
 (segment (start 38.1 25.4) (end 31.6 25.4) (width 0.65) (layer B.Cu) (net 9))
 (segment (start 63.5 43.18) (end 63.5 45.72) (width 0.65) (layer B.Cu) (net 9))
 (segment (start 60.96 40.64) (end 63.5 43.18) (width 0.65) (layer B.Cu) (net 9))
 (segment (start 54.61 31.75) (end 48.26 31.75) (width 0.65) (layer B.Cu) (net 9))
 (segment (start 46.99 33.02) (end 46.99 40.64) (width 0.65) (layer B.Cu) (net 9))
 (segment (start 58.42 27.94) (end 54.61 31.75) (width 0.65) (layer B.Cu) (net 9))
 (segment (start 48.26 31.75) (end 46.99 33.02) (width 0.65) (layer B.Cu) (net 9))
 (segment (start 46.99 40.64) (end 60.96 40.64) (width 0.65) (layer B.Cu) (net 9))
 (segment (start 66.04 48.26) (end 66.04 45.72) (width 0.65) (layer F.Cu) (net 19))
 (segment (start 91.44 48.26) (end 66.04 48.26) (width 0.65) (layer F.Cu) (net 19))
 (segment (start 91.44 39.37) (end 91.44 48.26) (width 0.65) (layer F.Cu) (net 19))
 (segment (start 88.9 39.37) (end 91.44 39.37) (width 0.65) (layer F.Cu) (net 19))
 (segment (start 88.9 33.02) (end 88.9 39.37) (width 0.65) (layer F.Cu) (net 19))
 (segment (start 71.12 27.94) (end 71.12 33.02) (width 0.65) (layer F.Cu) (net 19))
 (segment (start 71.12 33.02) (end 88.9 33.02) (width 0.65) (layer F.Cu) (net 19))
 (segment (start 68.58 40.64) (end 68.58 45.72) (width 0.65) (layer B.Cu) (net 15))
 (segment (start 50.8 35.56) (end 50.8 39.08291) (width 0.65) (layer B.Cu) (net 15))
 (segment (start 67.02291 39.08291) (end 68.58 40.64) (width 0.65) (layer B.Cu) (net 15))
 (segment (start 50.8 39.08291) (end 67.02291 39.08291) (width 0.65) (layer B.Cu) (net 15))
 (segment (start 70.83291 39.08291) (end 71.12 39.37) (width 0.65) (layer B.Cu) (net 17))
 (segment (start 69.6329 37.8829) (end 71.12 39.37) (width 0.65) (layer B.Cu) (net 17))
 (segment (start 53.34 35.56) (end 53.34 37.8829) (width 0.65) (layer B.Cu) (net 17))
 (segment (start 53.34 37.8829) (end 69.6329 37.8829) (width 0.65) (layer B.Cu) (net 17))
 (segment (start 71.12 39.37) (end 71.12 45.72) (width 0.65) (layer B.Cu) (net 17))
 (segment (start 73.66 35.56) (end 73.66 45.72) (width 0.65) (layer B.Cu) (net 22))
 (segment (start 76.2 35.56) (end 76.2 45.72) (width 0.65) (layer B.Cu) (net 23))
 (segment (start 78.74 35.56) (end 78.74 45.72) (width 0.65) (layer B.Cu) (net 25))
 (segment (start 83.82 35.56) (end 83.82 39.37) (width 0.65) (layer B.Cu) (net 29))
 (segment (start 81.28 41.91) (end 81.28 45.72) (width 0.65) (layer B.Cu) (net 29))
 (segment (start 83.82 39.37) (end 81.28 41.91) (width 0.65) (layer B.Cu) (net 29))
 (segment (start 82.55 31.75) (end 78.74 27.94) (width 0.65) (layer B.Cu) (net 18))
 (segment (start 83.82 41.91) (end 85.09 40.64) (width 0.65) (layer B.Cu) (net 18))
 (segment (start 83.82 45.72) (end 83.82 41.91) (width 0.65) (layer B.Cu) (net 18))
 (segment (start 85.09 40.64) (end 86.36 40.64) (width 0.65) (layer B.Cu) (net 18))
 (segment (start 86.36 40.64) (end 86.36 31.75) (width 0.65) (layer B.Cu) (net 18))
 (segment (start 86.36 31.75) (end 82.55 31.75) (width 0.65) (layer B.Cu) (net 18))
 (segment (start 87.63 30.48) (end 83.82 30.48) (width 0.65) (layer B.Cu) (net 16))
 (segment (start 83.82 30.48) (end 81.28 27.94) (width 0.65) (layer B.Cu) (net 16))
 (segment (start 87.63 41.91) (end 87.63 30.48) (width 0.65) (layer B.Cu) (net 16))
 (segment (start 86.36 45.72) (end 86.36 43.18) (width 0.65) (layer B.Cu) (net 16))
 (segment (start 86.36 43.18) (end 87.63 41.91) (width 0.65) (layer B.Cu) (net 16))
 (segment (start 88.9 40.64) (end 88.9 45.72) (width 0.65) (layer F.Cu) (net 27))
 (segment (start 81.28 35.56) (end 81.28 40.64) (width 0.65) (layer F.Cu) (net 27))
 (segment (start 81.28 40.64) (end 88.9 40.64) (width 0.65) (layer F.Cu) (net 27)))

